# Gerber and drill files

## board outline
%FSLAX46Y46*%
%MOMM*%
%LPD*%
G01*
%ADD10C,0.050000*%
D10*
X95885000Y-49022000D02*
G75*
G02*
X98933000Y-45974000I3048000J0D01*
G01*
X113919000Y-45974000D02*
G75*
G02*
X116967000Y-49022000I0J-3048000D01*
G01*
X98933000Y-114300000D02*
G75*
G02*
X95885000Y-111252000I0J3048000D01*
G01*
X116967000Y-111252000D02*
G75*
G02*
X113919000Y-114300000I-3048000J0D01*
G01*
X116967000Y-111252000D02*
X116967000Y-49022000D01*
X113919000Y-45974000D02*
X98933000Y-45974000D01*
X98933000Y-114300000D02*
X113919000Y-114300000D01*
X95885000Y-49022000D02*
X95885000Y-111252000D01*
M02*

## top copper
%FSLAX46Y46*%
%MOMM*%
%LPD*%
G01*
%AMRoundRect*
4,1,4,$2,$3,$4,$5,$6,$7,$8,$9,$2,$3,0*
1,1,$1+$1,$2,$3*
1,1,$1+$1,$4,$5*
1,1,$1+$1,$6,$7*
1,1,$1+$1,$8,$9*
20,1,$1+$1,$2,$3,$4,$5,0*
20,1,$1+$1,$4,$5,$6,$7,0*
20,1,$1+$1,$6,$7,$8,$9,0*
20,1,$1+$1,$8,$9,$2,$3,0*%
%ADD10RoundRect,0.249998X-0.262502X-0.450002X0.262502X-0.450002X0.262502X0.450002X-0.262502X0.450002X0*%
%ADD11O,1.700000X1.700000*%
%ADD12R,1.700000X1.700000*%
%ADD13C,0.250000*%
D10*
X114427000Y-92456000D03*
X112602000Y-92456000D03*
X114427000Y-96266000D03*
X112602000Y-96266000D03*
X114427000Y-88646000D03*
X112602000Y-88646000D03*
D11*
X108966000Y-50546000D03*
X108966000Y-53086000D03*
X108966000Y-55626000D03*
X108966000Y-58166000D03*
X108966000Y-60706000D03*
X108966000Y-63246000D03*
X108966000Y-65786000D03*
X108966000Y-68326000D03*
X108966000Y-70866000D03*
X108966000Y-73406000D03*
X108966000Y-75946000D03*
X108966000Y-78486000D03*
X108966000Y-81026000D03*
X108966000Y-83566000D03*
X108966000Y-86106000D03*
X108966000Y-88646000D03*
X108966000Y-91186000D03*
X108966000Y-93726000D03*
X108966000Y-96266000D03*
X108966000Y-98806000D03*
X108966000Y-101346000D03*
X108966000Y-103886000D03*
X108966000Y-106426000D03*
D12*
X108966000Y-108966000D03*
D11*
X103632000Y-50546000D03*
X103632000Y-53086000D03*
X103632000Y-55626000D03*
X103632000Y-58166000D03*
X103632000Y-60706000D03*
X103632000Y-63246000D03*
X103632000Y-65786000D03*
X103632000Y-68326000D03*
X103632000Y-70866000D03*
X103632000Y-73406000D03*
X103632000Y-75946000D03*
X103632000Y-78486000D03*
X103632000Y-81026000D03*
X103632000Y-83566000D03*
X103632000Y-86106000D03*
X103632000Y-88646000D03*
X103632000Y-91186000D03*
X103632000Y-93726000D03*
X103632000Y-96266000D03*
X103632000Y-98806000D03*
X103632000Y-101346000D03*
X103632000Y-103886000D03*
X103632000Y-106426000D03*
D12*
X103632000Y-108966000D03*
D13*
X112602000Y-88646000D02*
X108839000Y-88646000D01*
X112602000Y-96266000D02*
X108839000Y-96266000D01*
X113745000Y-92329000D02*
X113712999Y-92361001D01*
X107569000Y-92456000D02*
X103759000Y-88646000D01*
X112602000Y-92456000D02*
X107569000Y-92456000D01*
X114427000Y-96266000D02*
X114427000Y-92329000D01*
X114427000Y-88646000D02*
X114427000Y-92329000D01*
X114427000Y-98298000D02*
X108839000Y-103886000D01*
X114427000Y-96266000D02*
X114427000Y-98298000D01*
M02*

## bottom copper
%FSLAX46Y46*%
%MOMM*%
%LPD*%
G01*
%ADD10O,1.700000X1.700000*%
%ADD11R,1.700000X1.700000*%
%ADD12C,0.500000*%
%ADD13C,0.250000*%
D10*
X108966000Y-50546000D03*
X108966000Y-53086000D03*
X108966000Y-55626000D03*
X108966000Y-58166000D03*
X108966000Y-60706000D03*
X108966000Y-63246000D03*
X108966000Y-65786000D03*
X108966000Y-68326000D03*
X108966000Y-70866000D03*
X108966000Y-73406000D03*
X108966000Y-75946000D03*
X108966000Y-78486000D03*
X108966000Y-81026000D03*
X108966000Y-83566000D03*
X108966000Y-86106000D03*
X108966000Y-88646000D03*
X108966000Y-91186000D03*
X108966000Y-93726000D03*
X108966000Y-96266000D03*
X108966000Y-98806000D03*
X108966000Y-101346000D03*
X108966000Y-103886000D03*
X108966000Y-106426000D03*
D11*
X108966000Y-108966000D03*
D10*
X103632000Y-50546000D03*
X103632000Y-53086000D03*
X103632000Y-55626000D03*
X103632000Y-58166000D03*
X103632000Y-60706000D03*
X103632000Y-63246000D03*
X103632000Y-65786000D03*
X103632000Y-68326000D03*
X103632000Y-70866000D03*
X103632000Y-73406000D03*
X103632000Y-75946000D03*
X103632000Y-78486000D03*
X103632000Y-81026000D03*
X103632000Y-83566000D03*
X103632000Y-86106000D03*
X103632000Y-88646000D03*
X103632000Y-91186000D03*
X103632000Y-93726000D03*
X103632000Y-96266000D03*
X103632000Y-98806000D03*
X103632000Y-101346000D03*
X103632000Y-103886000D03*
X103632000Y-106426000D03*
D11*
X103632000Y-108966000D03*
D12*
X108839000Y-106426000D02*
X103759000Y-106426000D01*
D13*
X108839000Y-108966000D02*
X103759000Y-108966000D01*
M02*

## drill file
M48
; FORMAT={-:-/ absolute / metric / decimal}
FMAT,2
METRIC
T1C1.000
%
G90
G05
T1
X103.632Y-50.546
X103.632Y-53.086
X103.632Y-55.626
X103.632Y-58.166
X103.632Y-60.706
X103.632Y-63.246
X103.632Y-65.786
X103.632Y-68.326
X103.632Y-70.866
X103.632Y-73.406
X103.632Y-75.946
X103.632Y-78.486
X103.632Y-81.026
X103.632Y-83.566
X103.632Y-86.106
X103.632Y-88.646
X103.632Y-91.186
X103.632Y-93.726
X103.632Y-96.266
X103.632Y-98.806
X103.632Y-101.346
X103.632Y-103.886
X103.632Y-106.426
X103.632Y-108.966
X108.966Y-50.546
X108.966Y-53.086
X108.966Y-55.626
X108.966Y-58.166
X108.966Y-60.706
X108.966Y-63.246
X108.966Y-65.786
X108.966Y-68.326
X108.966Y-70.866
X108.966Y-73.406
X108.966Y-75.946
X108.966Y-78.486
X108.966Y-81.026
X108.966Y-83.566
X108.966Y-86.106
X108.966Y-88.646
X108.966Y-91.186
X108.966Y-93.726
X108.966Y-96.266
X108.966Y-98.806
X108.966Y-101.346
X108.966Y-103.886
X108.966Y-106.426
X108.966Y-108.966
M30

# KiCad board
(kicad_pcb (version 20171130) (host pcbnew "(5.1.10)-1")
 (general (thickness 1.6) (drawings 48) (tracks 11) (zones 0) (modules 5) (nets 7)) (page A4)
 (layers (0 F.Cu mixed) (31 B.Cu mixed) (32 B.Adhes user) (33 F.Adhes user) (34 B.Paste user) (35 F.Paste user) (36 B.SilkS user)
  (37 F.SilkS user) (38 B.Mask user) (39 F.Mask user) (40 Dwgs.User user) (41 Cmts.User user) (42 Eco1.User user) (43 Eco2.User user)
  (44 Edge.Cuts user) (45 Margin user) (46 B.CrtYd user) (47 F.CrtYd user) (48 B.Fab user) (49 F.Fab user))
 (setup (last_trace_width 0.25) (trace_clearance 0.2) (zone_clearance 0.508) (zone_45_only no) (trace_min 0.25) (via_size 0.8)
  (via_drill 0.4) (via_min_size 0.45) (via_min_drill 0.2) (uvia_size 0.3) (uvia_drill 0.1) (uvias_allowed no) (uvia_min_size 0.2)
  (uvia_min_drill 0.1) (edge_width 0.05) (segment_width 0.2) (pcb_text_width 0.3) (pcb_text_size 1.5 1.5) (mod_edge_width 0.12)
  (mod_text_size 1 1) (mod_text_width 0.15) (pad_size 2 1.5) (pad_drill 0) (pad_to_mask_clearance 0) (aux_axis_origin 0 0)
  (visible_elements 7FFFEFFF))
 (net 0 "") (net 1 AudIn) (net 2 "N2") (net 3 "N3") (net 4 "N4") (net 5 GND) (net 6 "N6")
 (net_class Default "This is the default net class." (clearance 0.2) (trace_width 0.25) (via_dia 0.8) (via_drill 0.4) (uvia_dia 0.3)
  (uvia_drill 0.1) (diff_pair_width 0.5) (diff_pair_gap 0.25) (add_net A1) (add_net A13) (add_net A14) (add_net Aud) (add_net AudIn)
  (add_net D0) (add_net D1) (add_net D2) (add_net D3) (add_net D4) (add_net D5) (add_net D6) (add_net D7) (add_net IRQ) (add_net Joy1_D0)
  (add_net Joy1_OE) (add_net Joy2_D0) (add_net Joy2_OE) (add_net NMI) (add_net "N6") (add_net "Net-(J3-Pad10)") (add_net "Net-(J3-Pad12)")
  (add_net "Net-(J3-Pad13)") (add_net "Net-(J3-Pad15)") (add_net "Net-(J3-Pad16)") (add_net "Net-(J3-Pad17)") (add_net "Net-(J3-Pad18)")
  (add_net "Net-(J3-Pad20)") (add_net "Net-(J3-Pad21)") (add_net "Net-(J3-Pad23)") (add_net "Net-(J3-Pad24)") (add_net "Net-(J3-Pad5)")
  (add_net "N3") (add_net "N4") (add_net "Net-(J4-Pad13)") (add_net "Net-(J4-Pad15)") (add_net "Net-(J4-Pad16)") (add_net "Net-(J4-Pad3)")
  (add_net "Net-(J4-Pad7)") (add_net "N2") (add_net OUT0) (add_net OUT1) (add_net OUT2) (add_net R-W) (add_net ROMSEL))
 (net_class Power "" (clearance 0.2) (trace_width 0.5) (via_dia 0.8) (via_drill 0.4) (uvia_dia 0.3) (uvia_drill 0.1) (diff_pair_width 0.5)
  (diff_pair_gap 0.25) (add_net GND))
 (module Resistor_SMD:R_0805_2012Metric (layer F.Cu) (at 113.5145 92.456)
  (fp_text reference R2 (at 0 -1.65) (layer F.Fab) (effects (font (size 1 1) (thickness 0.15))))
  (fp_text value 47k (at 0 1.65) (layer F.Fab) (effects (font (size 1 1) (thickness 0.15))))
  (pad 2 smd roundrect (at 0.9125 0) (size 1.025 1.4) (layers F.Cu F.Paste F.Mask) (roundrect_rratio 0.2439004878048781) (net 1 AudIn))
  (pad 1 smd roundrect (at -0.9125 0) (size 1.025 1.4) (layers F.Cu F.Paste F.Mask) (roundrect_rratio 0.2439004878048781) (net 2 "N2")))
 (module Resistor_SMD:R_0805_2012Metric (layer F.Cu) (at 113.5145 96.266)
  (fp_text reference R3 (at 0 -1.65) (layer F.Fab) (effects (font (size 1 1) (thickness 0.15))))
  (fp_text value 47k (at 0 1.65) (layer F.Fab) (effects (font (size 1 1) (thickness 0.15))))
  (pad 2 smd roundrect (at 0.9125 0) (size 1.025 1.4) (layers F.Cu F.Paste F.Mask) (roundrect_rratio 0.2439004878048781) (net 1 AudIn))
  (pad 1 smd roundrect (at -0.9125 0) (size 1.025 1.4) (layers F.Cu F.Paste F.Mask) (roundrect_rratio 0.2439004878048781) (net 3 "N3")))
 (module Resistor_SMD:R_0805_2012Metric (layer F.Cu) (at 113.5145 88.646)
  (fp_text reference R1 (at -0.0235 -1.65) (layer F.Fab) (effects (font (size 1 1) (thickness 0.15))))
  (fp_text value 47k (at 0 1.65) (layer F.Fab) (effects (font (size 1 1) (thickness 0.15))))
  (pad 2 smd roundrect (at 0.9125 0) (size 1.025 1.4) (layers F.Cu F.Paste F.Mask) (roundrect_rratio 0.2439004878048781) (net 1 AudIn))
  (pad 1 smd roundrect (at -0.9125 0) (size 1.025 1.4) (layers F.Cu F.Paste F.Mask) (roundrect_rratio 0.2439004878048781) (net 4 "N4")))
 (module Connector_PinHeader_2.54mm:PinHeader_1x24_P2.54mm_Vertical (layer B.Cu) (at 108.966 108.966)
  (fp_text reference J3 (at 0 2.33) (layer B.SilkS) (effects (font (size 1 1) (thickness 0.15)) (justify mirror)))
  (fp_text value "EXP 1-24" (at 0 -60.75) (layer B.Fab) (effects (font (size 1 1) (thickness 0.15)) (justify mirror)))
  (pad 24 thru_hole oval (at 0 -58.42) (size 1.7 1.7) (drill 1) (layers *.Cu *.Mask))
  (pad 23 thru_hole oval (at 0 -55.88) (size 1.7 1.7) (drill 1) (layers *.Cu *.Mask))
  (pad 22 thru_hole oval (at 0 -53.34) (size 1.7 1.7) (drill 1) (layers *.Cu *.Mask))
  (pad 21 thru_hole oval (at 0 -50.8) (size 1.7 1.7) (drill 1) (layers *.Cu *.Mask))
  (pad 20 thru_hole oval (at 0 -48.26) (size 1.7 1.7) (drill 1) (layers *.Cu *.Mask))
  (pad 19 thru_hole oval (at 0 -45.72) (size 1.7 1.7) (drill 1) (layers *.Cu *.Mask))
  (pad 18 thru_hole oval (at 0 -43.18) (size 1.7 1.7) (drill 1) (layers *.Cu *.Mask))
  (pad 17 thru_hole oval (at 0 -40.64) (size 1.7 1.7) (drill 1) (layers *.Cu *.Mask))
  (pad 16 thru_hole oval (at 0 -38.1) (size 1.7 1.7) (drill 1) (layers *.Cu *.Mask))
  (pad 15 thru_hole oval (at 0 -35.56) (size 1.7 1.7) (drill 1) (layers *.Cu *.Mask))
  (pad 14 thru_hole oval (at 0 -33.02) (size 1.7 1.7) (drill 1) (layers *.Cu *.Mask))
  (pad 13 thru_hole oval (at 0 -30.48) (size 1.7 1.7) (drill 1) (layers *.Cu *.Mask))
  (pad 12 thru_hole oval (at 0 -27.94) (size 1.7 1.7) (drill 1) (layers *.Cu *.Mask))
  (pad 11 thru_hole oval (at 0 -25.4) (size 1.7 1.7) (drill 1) (layers *.Cu *.Mask))
  (pad 10 thru_hole oval (at 0 -22.86) (size 1.7 1.7) (drill 1) (layers *.Cu *.Mask))
  (pad 9 thru_hole oval (at 0 -20.32) (size 1.7 1.7) (drill 1) (layers *.Cu *.Mask) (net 4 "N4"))
  (pad 8 thru_hole oval (at 0 -17.78) (size 1.7 1.7) (drill 1) (layers *.Cu *.Mask))
  (pad 7 thru_hole oval (at 0 -15.24) (size 1.7 1.7) (drill 1) (layers *.Cu *.Mask))
  (pad 6 thru_hole oval (at 0 -12.7) (size 1.7 1.7) (drill 1) (layers *.Cu *.Mask) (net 3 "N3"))
  (pad 5 thru_hole oval (at 0 -10.16) (size 1.7 1.7) (drill 1) (layers *.Cu *.Mask))
  (pad 4 thru_hole oval (at 0 -7.62) (size 1.7 1.7) (drill 1) (layers *.Cu *.Mask))
  (pad 3 thru_hole oval (at 0 -5.08) (size 1.7 1.7) (drill 1) (layers *.Cu *.Mask) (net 1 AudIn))
  (pad 2 thru_hole oval (at 0 -2.54) (size 1.7 1.7) (drill 1) (layers *.Cu *.Mask) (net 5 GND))
  (pad 1 thru_hole rect (at 0 0) (size 1.7 1.7) (drill 1) (layers *.Cu *.Mask) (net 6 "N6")))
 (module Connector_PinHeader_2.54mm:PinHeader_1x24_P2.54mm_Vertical (layer B.Cu) (at 103.632 108.966)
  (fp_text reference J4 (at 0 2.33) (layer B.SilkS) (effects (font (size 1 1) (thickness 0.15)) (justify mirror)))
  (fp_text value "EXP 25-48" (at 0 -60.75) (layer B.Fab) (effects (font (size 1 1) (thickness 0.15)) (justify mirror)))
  (pad 24 thru_hole oval (at 0 -58.42) (size 1.7 1.7) (drill 1) (layers *.Cu *.Mask))
  (pad 23 thru_hole oval (at 0 -55.88) (size 1.7 1.7) (drill 1) (layers *.Cu *.Mask))
  (pad 22 thru_hole oval (at 0 -53.34) (size 1.7 1.7) (drill 1) (layers *.Cu *.Mask))
  (pad 21 thru_hole oval (at 0 -50.8) (size 1.7 1.7) (drill 1) (layers *.Cu *.Mask))
  (pad 20 thru_hole oval (at 0 -48.26) (size 1.7 1.7) (drill 1) (layers *.Cu *.Mask))
  (pad 19 thru_hole oval (at 0 -45.72) (size 1.7 1.7) (drill 1) (layers *.Cu *.Mask))
  (pad 18 thru_hole oval (at 0 -43.18) (size 1.7 1.7) (drill 1) (layers *.Cu *.Mask))
  (pad 17 thru_hole oval (at 0 -40.64) (size 1.7 1.7) (drill 1) (layers *.Cu *.Mask))
  (pad 16 thru_hole oval (at 0 -38.1) (size 1.7 1.7) (drill 1) (layers *.Cu *.Mask))
  (pad 15 thru_hole oval (at 0 -35.56) (size 1.7 1.7) (drill 1) (layers *.Cu *.Mask))
  (pad 14 thru_hole oval (at 0 -33.02) (size 1.7 1.7) (drill 1) (layers *.Cu *.Mask))
  (pad 13 thru_hole oval (at 0 -30.48) (size 1.7 1.7) (drill 1) (layers *.Cu *.Mask))
  (pad 12 thru_hole oval (at 0 -27.94) (size 1.7 1.7) (drill 1) (layers *.Cu *.Mask))
  (pad 11 thru_hole oval (at 0 -25.4) (size 1.7 1.7) (drill 1) (layers *.Cu *.Mask))
  (pad 10 thru_hole oval (at 0 -22.86) (size 1.7 1.7) (drill 1) (layers *.Cu *.Mask))
  (pad 9 thru_hole oval (at 0 -20.32) (size 1.7 1.7) (drill 1) (layers *.Cu *.Mask) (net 2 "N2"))
  (pad 8 thru_hole oval (at 0 -17.78) (size 1.7 1.7) (drill 1) (layers *.Cu *.Mask))
  (pad 7 thru_hole oval (at 0 -15.24) (size 1.7 1.7) (drill 1) (layers *.Cu *.Mask))
  (pad 6 thru_hole oval (at 0 -12.7) (size 1.7 1.7) (drill 1) (layers *.Cu *.Mask))
  (pad 5 thru_hole oval (at 0 -10.16) (size 1.7 1.7) (drill 1) (layers *.Cu *.Mask))
  (pad 4 thru_hole oval (at 0 -7.62) (size 1.7 1.7) (drill 1) (layers *.Cu *.Mask))
  (pad 3 thru_hole oval (at 0 -5.08) (size 1.7 1.7) (drill 1) (layers *.Cu *.Mask))
  (pad 2 thru_hole oval (at 0 -2.54) (size 1.7 1.7) (drill 1) (layers *.Cu *.Mask) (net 5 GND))
  (pad 1 thru_hole rect (at 0 0) (size 1.7 1.7) (drill 1) (layers *.Cu *.Mask) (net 6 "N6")))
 (gr_arc (start 98.933 49.022) (end 98.933 45.974) (angle -90) (layer Edge.Cuts) (width 0.05))
 (gr_arc (start 113.919 49.022) (end 116.967 49.022) (angle -90) (layer Edge.Cuts) (width 0.05))
 (gr_arc (start 98.933 111.252) (end 95.885 111.252) (angle -90) (layer Edge.Cuts) (width 0.05))
 (gr_arc (start 113.919 111.252) (end 113.919 114.3) (angle -90) (layer Edge.Cuts) (width 0.05))
 (gr_line (start 116.967 111.252) (end 116.967 49.022) (layer Edge.Cuts) (width 0.05))
 (gr_line (start 113.919 45.974) (end 98.933 45.974) (layer Edge.Cuts) (width 0.05))
 (gr_line (start 98.933 114.3) (end 113.919 114.3) (layer Edge.Cuts) (width 0.05))
 (gr_line (start 95.885 49.022) (end 95.885 111.252) (layer Edge.Cuts) (width 0.05))
 (segment (start 108.839 106.426) (end 103.759 106.426) (width 0.5) (layer B.Cu) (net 5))
 (segment (start 112.602 88.646) (end 108.839 88.646) (width 0.25) (layer F.Cu) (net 4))
 (segment (start 112.602 96.266) (end 108.839 96.266) (width 0.25) (layer F.Cu) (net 3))
 (segment (start 113.745 92.329) (end 113.712999 92.361001) (width 0.25) (layer F.Cu) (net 2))
 (segment (start 107.569 92.456) (end 103.759 88.646) (width 0.25) (layer F.Cu) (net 2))
 (segment (start 112.602 92.456) (end 107.569 92.456) (width 0.25) (layer F.Cu) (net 2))
 (segment (start 114.427 96.266) (end 114.427 92.329) (width 0.25) (layer F.Cu) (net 1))
 (segment (start 114.427 88.646) (end 114.427 92.329) (width 0.25) (layer F.Cu) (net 1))
 (segment (start 114.427 98.298) (end 108.839 103.886) (width 0.25) (layer F.Cu) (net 1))
 (segment (start 114.427 96.266) (end 114.427 98.298) (width 0.25) (layer F.Cu) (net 1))
 (segment (start 108.839 108.966) (end 103.759 108.966) (width 0.25) (layer B.Cu) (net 6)))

